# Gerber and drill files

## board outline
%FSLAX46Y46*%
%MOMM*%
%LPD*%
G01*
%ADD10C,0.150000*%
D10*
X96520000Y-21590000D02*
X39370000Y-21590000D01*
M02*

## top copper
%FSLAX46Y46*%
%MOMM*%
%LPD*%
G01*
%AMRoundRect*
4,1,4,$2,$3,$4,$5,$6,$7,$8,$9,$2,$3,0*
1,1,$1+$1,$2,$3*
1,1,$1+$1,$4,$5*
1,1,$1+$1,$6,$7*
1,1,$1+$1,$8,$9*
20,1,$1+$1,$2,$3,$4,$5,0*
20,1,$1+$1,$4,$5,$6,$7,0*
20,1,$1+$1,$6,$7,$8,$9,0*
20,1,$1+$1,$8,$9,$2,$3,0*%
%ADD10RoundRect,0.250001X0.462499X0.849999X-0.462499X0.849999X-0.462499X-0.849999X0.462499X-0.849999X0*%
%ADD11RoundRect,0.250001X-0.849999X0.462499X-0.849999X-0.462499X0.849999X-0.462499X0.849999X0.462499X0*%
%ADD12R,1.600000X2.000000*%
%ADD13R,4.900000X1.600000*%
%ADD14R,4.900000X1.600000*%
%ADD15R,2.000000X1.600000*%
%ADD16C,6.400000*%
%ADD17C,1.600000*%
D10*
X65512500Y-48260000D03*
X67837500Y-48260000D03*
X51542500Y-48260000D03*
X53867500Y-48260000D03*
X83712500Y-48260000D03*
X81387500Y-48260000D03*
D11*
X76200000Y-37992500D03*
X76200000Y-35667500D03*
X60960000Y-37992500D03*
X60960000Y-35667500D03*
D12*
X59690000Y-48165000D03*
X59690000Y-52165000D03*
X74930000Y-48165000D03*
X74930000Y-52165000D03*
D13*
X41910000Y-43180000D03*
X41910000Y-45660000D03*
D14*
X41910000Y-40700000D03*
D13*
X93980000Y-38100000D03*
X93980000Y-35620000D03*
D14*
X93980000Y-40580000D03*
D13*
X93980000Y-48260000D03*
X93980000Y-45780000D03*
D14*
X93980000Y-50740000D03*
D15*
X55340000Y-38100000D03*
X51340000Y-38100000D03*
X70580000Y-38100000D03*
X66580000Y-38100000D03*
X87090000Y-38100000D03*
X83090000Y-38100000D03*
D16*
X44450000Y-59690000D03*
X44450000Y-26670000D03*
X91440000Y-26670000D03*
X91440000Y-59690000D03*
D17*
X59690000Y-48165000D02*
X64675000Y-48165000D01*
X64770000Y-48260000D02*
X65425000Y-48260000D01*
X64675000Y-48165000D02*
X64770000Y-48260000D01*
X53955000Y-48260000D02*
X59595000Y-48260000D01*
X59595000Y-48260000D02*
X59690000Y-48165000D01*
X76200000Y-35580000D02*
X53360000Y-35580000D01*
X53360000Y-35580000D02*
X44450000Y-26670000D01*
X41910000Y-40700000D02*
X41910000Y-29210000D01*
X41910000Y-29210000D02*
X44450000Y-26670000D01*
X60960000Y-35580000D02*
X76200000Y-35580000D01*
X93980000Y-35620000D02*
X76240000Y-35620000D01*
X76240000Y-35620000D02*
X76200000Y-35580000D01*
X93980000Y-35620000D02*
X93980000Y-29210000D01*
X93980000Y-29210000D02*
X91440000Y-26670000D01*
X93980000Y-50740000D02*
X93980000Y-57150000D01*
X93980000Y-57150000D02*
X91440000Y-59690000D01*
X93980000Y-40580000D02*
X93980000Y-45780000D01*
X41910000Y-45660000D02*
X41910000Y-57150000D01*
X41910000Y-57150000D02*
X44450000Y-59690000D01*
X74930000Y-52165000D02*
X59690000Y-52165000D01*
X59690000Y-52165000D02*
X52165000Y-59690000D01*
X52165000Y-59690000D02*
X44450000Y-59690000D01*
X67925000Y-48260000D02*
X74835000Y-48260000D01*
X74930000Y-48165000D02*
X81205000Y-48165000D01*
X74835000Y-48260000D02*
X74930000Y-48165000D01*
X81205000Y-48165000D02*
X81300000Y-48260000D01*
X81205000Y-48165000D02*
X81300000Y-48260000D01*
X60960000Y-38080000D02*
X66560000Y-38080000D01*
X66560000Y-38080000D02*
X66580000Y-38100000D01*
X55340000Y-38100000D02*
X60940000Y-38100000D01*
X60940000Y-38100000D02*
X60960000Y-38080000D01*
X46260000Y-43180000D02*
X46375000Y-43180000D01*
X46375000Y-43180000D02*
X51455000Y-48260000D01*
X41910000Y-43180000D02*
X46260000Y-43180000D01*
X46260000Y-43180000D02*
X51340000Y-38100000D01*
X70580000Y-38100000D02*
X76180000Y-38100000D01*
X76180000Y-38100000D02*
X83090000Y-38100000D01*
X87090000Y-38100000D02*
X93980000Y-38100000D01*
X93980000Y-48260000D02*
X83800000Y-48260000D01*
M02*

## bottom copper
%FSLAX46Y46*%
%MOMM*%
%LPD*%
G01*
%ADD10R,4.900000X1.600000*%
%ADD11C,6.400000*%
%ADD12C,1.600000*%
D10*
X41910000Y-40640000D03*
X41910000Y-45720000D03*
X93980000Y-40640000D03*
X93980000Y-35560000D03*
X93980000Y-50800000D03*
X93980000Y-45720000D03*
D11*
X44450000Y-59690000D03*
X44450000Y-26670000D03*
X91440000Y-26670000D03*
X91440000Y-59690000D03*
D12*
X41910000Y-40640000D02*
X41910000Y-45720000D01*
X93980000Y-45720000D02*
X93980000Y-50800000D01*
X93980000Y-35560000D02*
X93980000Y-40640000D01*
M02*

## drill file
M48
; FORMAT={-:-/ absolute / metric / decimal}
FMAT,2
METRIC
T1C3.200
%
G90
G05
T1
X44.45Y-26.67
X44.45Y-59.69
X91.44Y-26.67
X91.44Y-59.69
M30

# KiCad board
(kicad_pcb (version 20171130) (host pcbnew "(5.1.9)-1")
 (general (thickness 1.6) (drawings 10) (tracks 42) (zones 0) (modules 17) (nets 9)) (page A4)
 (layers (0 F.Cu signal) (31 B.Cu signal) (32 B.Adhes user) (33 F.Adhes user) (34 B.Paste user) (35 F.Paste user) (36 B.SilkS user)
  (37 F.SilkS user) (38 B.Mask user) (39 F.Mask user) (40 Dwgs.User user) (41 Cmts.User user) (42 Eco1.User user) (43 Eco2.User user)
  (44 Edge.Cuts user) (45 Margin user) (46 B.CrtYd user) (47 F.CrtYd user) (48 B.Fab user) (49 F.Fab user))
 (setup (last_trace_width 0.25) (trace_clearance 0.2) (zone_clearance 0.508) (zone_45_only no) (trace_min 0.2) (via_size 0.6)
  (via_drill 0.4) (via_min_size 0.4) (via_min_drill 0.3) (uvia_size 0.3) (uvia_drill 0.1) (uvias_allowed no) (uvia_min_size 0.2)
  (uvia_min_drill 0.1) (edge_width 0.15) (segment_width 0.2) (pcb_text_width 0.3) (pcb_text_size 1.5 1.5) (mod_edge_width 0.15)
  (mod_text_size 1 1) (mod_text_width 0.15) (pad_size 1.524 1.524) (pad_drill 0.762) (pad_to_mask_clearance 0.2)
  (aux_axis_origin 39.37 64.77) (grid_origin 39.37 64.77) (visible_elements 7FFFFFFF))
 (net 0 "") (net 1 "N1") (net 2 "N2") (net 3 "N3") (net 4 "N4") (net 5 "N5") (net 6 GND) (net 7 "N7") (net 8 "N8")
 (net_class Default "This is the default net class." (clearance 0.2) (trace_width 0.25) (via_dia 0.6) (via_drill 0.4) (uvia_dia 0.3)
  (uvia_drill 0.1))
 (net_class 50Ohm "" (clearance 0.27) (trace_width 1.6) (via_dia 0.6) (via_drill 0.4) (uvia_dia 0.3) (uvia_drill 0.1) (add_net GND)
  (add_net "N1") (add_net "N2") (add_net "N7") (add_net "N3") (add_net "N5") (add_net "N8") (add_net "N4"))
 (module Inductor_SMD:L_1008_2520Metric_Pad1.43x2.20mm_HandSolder (layer F.Cu) (at 66.675 48.26 180)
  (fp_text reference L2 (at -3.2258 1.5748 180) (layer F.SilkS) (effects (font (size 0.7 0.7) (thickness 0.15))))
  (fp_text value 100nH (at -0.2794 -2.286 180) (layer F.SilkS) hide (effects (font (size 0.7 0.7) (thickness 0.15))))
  (pad 2 smd roundrect (at 1.1625 0 180) (size 1.425 2.2) (layers F.Cu F.Paste F.Mask) (roundrect_rratio 0.175439) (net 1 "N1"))
  (pad 1 smd roundrect (at -1.1625 0 180) (size 1.425 2.2) (layers F.Cu F.Paste F.Mask) (roundrect_rratio 0.175439) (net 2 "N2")))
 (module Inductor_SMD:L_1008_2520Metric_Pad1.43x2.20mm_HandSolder (layer F.Cu) (at 52.705 48.26 180)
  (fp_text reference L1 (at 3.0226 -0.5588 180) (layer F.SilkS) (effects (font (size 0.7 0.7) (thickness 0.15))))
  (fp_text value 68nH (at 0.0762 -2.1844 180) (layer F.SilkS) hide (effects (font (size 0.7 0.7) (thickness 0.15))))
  (pad 2 smd roundrect (at 1.1625 0 180) (size 1.425 2.2) (layers F.Cu F.Paste F.Mask) (roundrect_rratio 0.175439) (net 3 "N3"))
  (pad 1 smd roundrect (at -1.1625 0 180) (size 1.425 2.2) (layers F.Cu F.Paste F.Mask) (roundrect_rratio 0.175439) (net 1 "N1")))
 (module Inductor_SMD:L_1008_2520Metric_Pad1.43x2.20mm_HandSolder (layer F.Cu) (at 82.55 48.26 180)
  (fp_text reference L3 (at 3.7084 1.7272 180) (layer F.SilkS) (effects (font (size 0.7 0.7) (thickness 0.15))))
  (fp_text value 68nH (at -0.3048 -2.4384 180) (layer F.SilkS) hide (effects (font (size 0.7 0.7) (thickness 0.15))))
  (pad 1 smd roundrect (at -1.1625 0 180) (size 1.425 2.2) (layers F.Cu F.Paste F.Mask) (roundrect_rratio 0.175439) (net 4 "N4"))
  (pad 2 smd roundrect (at 1.1625 0 180) (size 1.425 2.2) (layers F.Cu F.Paste F.Mask) (roundrect_rratio 0.175439) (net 2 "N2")))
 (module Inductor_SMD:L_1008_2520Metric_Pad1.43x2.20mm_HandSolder (layer F.Cu) (at 76.2 36.83 270)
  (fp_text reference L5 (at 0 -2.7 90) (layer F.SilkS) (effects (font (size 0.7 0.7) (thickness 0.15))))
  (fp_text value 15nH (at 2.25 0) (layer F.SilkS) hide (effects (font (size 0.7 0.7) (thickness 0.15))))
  (pad 2 smd roundrect (at 1.1625 0 270) (size 1.425 2.2) (layers F.Cu F.Paste F.Mask) (roundrect_rratio 0.175439) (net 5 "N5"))
  (pad 1 smd roundrect (at -1.1625 0 270) (size 1.425 2.2) (layers F.Cu F.Paste F.Mask) (roundrect_rratio 0.175439) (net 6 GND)))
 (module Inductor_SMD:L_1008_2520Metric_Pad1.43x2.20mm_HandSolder (layer F.Cu) (at 60.96 36.83 270)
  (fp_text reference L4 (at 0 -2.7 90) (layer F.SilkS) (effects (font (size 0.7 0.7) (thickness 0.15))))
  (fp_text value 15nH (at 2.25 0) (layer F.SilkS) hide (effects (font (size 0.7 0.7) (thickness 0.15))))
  (pad 2 smd roundrect (at 1.1625 0 270) (size 1.425 2.2) (layers F.Cu F.Paste F.Mask) (roundrect_rratio 0.175439) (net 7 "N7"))
  (pad 1 smd roundrect (at -1.1625 0 270) (size 1.425 2.2) (layers F.Cu F.Paste F.Mask) (roundrect_rratio 0.175439) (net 6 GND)))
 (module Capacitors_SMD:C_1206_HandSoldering (layer F.Cu) (at 59.69 50.165 270)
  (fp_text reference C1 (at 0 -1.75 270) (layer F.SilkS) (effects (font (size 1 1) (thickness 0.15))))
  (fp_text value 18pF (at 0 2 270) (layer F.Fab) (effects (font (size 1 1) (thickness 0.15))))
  (pad 1 smd rect (at -2 0 270) (size 2 1.6) (layers F.Cu F.Paste F.Mask) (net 1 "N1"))
  (pad 2 smd rect (at 2 0 270) (size 2 1.6) (layers F.Cu F.Paste F.Mask) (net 6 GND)))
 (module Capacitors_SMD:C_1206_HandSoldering (layer F.Cu) (at 74.93 50.165 270)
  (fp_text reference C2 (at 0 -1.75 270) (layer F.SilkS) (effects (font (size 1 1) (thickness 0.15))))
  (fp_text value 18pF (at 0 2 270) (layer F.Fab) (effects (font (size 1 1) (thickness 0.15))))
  (pad 1 smd rect (at -2 0 270) (size 2 1.6) (layers F.Cu F.Paste F.Mask) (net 2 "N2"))
  (pad 2 smd rect (at 2 0 270) (size 2 1.6) (layers F.Cu F.Paste F.Mask) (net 6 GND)))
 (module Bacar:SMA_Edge (layer F.Cu) (at 41.91 43.18 90)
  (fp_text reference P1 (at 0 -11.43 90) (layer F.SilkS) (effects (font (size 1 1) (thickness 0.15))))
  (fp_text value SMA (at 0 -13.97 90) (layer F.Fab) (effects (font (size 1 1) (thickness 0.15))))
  (pad 1 connect rect (at 0 0 90) (size 1.6 4.9) (layers F.Cu F.Mask) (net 3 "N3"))
  (pad 2 connect rect (at -2.48 0 90) (size 1.6 4.9) (layers F.Cu F.Mask) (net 6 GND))
  (pad 2 smd rect (at 2.48 0 90) (size 1.6 4.9) (layers F.Cu F.Paste F.Mask) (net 6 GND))
  (pad 2 smd rect (at 2.54 0 90) (size 1.6 4.9) (layers B.Cu F.Paste F.Mask) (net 6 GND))
  (pad 2 smd rect (at -2.54 0 90) (size 1.6 4.9) (layers B.Cu F.Paste F.Mask) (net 6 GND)))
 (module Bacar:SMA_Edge (layer F.Cu) (at 93.98 38.1 270)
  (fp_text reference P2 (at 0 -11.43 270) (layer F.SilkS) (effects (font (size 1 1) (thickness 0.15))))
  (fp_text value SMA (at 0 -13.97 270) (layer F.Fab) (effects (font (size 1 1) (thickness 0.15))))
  (pad 1 connect rect (at 0 0 270) (size 1.6 4.9) (layers F.Cu F.Mask) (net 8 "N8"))
  (pad 2 connect rect (at -2.48 0 270) (size 1.6 4.9) (layers F.Cu F.Mask) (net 6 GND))
  (pad 2 smd rect (at 2.48 0 270) (size 1.6 4.9) (layers F.Cu F.Paste F.Mask) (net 6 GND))
  (pad 2 smd rect (at 2.54 0 270) (size 1.6 4.9) (layers B.Cu F.Paste F.Mask) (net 6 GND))
  (pad 2 smd rect (at -2.54 0 270) (size 1.6 4.9) (layers B.Cu F.Paste F.Mask) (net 6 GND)))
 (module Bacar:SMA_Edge (layer F.Cu) (at 93.98 48.26 270)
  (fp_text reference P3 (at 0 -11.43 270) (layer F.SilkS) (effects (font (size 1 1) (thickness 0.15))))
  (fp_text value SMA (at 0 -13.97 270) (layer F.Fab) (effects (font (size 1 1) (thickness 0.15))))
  (pad 1 connect rect (at 0 0 270) (size 1.6 4.9) (layers F.Cu F.Mask) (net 4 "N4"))
  (pad 2 connect rect (at -2.48 0 270) (size 1.6 4.9) (layers F.Cu F.Mask) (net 6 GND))
  (pad 2 smd rect (at 2.48 0 270) (size 1.6 4.9) (layers F.Cu F.Paste F.Mask) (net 6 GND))
  (pad 2 smd rect (at 2.54 0 270) (size 1.6 4.9) (layers B.Cu F.Paste F.Mask) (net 6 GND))
  (pad 2 smd rect (at -2.54 0 270) (size 1.6 4.9) (layers B.Cu F.Paste F.Mask) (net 6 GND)))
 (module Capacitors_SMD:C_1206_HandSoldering (layer F.Cu) (at 53.34 38.1 180)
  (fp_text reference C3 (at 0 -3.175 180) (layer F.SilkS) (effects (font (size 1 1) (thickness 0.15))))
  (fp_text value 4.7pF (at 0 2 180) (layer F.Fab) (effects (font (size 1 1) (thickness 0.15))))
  (pad 1 smd rect (at -2 0 180) (size 2 1.6) (layers F.Cu F.Paste F.Mask) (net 7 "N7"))
  (pad 2 smd rect (at 2 0 180) (size 2 1.6) (layers F.Cu F.Paste F.Mask) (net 3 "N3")))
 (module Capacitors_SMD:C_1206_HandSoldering (layer F.Cu) (at 68.58 38.1 180)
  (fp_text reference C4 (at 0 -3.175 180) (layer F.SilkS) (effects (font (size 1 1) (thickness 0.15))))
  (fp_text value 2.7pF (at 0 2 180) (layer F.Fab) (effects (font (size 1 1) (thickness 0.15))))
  (pad 1 smd rect (at -2 0 180) (size 2 1.6) (layers F.Cu F.Paste F.Mask) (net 5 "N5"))
  (pad 2 smd rect (at 2 0 180) (size 2 1.6) (layers F.Cu F.Paste F.Mask) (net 7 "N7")))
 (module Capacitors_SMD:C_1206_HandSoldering (layer F.Cu) (at 85.09 38.1 180)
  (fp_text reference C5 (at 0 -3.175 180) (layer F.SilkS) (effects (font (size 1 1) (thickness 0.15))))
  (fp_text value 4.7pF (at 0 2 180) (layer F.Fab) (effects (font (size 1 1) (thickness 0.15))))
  (pad 1 smd rect (at -2 0 180) (size 2 1.6) (layers F.Cu F.Paste F.Mask) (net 8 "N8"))
  (pad 2 smd rect (at 2 0 180) (size 2 1.6) (layers F.Cu F.Paste F.Mask) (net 5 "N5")))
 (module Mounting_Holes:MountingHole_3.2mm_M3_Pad (layer F.Cu) (at 44.45 59.69)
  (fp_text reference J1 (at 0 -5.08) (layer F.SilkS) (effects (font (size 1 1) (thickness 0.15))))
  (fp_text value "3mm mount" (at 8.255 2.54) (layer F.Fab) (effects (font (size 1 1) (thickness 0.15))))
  (pad 1 thru_hole circle (at 0 0) (size 6.4 6.4) (drill 3.2) (layers *.Cu *.Mask) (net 6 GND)))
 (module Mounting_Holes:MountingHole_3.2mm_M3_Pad (layer F.Cu) (at 44.45 26.67)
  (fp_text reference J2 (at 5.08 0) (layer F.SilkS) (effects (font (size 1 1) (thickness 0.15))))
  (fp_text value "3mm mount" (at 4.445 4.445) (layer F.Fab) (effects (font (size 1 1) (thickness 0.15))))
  (pad 1 thru_hole circle (at 0 0) (size 6.4 6.4) (drill 3.2) (layers *.Cu *.Mask) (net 6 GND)))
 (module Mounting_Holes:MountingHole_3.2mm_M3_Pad (layer F.Cu) (at 91.44 26.67)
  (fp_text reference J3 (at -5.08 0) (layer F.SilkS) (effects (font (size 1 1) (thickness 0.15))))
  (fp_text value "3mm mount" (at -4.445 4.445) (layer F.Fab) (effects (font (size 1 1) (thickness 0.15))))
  (pad 1 thru_hole circle (at 0 0) (size 6.4 6.4) (drill 3.2) (layers *.Cu *.Mask) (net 6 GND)))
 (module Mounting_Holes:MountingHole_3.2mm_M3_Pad (layer F.Cu) (at 91.44 59.69)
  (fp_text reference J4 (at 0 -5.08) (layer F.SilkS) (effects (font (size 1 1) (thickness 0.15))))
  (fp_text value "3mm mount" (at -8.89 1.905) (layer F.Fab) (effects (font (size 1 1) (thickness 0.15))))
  (pad 1 thru_hole circle (at 0 0) (size 6.4 6.4) (drill 3.2) (layers *.Cu *.Mask) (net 6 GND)))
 (gr_line (start 96.52 21.59) (end 39.37 21.59) (angle 90) (layer Edge.Cuts) (width 0.15))
 (segment (start 59.69 48.165) (end 64.675 48.165) (width 1.6) (layer F.Cu) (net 1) (status 400000))
 (segment (start 64.77 48.26) (end 65.425 48.26) (width 1.6) (layer F.Cu) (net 1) (status 800000))
 (segment (start 64.675 48.165) (end 64.77 48.26) (width 1.6) (layer F.Cu) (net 1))
 (segment (start 53.955 48.26) (end 59.595 48.26) (width 1.6) (layer F.Cu) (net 1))
 (segment (start 59.595 48.26) (end 59.69 48.165) (width 1.6) (layer F.Cu) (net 1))
 (segment (start 76.2 35.58) (end 53.36 35.58) (width 1.6) (layer F.Cu) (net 6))
 (segment (start 53.36 35.58) (end 44.45 26.67) (width 1.6) (layer F.Cu) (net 6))
 (segment (start 41.91 40.7) (end 41.91 29.21) (width 1.6) (layer F.Cu) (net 6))
 (segment (start 41.91 29.21) (end 44.45 26.67) (width 1.6) (layer F.Cu) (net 6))
 (segment (start 41.91 40.64) (end 41.91 45.72) (width 1.6) (layer B.Cu) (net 6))
 (segment (start 93.98 45.72) (end 93.98 50.8) (width 1.6) (layer B.Cu) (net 6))
 (segment (start 93.98 35.56) (end 93.98 40.64) (width 1.6) (layer B.Cu) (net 6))
 (segment (start 60.96 35.58) (end 76.2 35.58) (width 1.6) (layer F.Cu) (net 6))
 (segment (start 93.98 35.62) (end 76.24 35.62) (width 1.6) (layer F.Cu) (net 6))
 (segment (start 76.24 35.62) (end 76.2 35.58) (width 1.6) (layer F.Cu) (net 6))
 (segment (start 93.98 35.62) (end 93.98 29.21) (width 1.6) (layer F.Cu) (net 6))
 (segment (start 93.98 29.21) (end 91.44 26.67) (width 1.6) (layer F.Cu) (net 6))
 (segment (start 93.98 50.74) (end 93.98 57.15) (width 1.6) (layer F.Cu) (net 6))
 (segment (start 93.98 57.15) (end 91.44 59.69) (width 1.6) (layer F.Cu) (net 6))
 (segment (start 93.98 40.58) (end 93.98 45.78) (width 1.6) (layer F.Cu) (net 6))
 (segment (start 41.91 45.66) (end 41.91 57.15) (width 1.6) (layer F.Cu) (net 6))
 (segment (start 41.91 57.15) (end 44.45 59.69) (width 1.6) (layer F.Cu) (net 6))
 (segment (start 74.93 52.165) (end 59.69 52.165) (width 1.6) (layer F.Cu) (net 6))
 (segment (start 59.69 52.165) (end 52.165 59.69) (width 1.6) (layer F.Cu) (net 6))
 (segment (start 52.165 59.69) (end 44.45 59.69) (width 1.6) (layer F.Cu) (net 6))
 (segment (start 67.925 48.26) (end 74.835 48.26) (width 1.6) (layer F.Cu) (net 2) (status C00000))
 (segment (start 74.93 48.165) (end 81.205 48.165) (width 1.6) (layer F.Cu) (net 2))
 (segment (start 74.835 48.26) (end 74.93 48.165) (width 1.6) (layer F.Cu) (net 2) (status C00000))
 (segment (start 81.205 48.165) (end 81.3 48.26) (width 1.6) (layer F.Cu) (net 2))
 (segment (start 81.205 48.165) (end 81.3 48.26) (width 1.6) (layer F.Cu) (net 2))
 (segment (start 60.96 38.08) (end 66.56 38.08) (width 1.6) (layer F.Cu) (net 7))
 (segment (start 66.56 38.08) (end 66.58 38.1) (width 1.6) (layer F.Cu) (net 7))
 (segment (start 55.34 38.1) (end 60.94 38.1) (width 1.6) (layer F.Cu) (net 7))
 (segment (start 60.94 38.1) (end 60.96 38.08) (width 1.6) (layer F.Cu) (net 7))
 (segment (start 46.26 43.18) (end 46.375 43.18) (width 1.6) (layer F.Cu) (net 3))
 (segment (start 46.375 43.18) (end 51.455 48.26) (width 1.6) (layer F.Cu) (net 3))
 (segment (start 41.91 43.18) (end 46.26 43.18) (width 1.6) (layer F.Cu) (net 3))
 (segment (start 46.26 43.18) (end 51.34 38.1) (width 1.6) (layer F.Cu) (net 3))
 (segment (start 70.58 38.1) (end 76.18 38.1) (width 1.6) (layer F.Cu) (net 5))
 (segment (start 76.18 38.1) (end 83.09 38.1) (width 1.6) (layer F.Cu) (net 5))
 (segment (start 87.09 38.1) (end 93.98 38.1) (width 1.6) (layer F.Cu) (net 8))
 (segment (start 93.98 48.26) (end 83.8 48.26) (width 1.6) (layer F.Cu) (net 4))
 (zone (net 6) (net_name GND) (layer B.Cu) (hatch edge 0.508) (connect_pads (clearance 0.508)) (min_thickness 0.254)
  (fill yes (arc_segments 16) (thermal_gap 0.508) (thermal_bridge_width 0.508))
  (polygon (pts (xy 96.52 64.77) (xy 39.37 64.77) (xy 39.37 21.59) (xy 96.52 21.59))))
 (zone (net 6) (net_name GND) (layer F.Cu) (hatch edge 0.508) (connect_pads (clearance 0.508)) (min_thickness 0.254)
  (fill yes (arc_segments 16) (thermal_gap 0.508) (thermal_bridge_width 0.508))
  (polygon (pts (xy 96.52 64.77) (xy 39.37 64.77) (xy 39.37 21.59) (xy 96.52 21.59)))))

